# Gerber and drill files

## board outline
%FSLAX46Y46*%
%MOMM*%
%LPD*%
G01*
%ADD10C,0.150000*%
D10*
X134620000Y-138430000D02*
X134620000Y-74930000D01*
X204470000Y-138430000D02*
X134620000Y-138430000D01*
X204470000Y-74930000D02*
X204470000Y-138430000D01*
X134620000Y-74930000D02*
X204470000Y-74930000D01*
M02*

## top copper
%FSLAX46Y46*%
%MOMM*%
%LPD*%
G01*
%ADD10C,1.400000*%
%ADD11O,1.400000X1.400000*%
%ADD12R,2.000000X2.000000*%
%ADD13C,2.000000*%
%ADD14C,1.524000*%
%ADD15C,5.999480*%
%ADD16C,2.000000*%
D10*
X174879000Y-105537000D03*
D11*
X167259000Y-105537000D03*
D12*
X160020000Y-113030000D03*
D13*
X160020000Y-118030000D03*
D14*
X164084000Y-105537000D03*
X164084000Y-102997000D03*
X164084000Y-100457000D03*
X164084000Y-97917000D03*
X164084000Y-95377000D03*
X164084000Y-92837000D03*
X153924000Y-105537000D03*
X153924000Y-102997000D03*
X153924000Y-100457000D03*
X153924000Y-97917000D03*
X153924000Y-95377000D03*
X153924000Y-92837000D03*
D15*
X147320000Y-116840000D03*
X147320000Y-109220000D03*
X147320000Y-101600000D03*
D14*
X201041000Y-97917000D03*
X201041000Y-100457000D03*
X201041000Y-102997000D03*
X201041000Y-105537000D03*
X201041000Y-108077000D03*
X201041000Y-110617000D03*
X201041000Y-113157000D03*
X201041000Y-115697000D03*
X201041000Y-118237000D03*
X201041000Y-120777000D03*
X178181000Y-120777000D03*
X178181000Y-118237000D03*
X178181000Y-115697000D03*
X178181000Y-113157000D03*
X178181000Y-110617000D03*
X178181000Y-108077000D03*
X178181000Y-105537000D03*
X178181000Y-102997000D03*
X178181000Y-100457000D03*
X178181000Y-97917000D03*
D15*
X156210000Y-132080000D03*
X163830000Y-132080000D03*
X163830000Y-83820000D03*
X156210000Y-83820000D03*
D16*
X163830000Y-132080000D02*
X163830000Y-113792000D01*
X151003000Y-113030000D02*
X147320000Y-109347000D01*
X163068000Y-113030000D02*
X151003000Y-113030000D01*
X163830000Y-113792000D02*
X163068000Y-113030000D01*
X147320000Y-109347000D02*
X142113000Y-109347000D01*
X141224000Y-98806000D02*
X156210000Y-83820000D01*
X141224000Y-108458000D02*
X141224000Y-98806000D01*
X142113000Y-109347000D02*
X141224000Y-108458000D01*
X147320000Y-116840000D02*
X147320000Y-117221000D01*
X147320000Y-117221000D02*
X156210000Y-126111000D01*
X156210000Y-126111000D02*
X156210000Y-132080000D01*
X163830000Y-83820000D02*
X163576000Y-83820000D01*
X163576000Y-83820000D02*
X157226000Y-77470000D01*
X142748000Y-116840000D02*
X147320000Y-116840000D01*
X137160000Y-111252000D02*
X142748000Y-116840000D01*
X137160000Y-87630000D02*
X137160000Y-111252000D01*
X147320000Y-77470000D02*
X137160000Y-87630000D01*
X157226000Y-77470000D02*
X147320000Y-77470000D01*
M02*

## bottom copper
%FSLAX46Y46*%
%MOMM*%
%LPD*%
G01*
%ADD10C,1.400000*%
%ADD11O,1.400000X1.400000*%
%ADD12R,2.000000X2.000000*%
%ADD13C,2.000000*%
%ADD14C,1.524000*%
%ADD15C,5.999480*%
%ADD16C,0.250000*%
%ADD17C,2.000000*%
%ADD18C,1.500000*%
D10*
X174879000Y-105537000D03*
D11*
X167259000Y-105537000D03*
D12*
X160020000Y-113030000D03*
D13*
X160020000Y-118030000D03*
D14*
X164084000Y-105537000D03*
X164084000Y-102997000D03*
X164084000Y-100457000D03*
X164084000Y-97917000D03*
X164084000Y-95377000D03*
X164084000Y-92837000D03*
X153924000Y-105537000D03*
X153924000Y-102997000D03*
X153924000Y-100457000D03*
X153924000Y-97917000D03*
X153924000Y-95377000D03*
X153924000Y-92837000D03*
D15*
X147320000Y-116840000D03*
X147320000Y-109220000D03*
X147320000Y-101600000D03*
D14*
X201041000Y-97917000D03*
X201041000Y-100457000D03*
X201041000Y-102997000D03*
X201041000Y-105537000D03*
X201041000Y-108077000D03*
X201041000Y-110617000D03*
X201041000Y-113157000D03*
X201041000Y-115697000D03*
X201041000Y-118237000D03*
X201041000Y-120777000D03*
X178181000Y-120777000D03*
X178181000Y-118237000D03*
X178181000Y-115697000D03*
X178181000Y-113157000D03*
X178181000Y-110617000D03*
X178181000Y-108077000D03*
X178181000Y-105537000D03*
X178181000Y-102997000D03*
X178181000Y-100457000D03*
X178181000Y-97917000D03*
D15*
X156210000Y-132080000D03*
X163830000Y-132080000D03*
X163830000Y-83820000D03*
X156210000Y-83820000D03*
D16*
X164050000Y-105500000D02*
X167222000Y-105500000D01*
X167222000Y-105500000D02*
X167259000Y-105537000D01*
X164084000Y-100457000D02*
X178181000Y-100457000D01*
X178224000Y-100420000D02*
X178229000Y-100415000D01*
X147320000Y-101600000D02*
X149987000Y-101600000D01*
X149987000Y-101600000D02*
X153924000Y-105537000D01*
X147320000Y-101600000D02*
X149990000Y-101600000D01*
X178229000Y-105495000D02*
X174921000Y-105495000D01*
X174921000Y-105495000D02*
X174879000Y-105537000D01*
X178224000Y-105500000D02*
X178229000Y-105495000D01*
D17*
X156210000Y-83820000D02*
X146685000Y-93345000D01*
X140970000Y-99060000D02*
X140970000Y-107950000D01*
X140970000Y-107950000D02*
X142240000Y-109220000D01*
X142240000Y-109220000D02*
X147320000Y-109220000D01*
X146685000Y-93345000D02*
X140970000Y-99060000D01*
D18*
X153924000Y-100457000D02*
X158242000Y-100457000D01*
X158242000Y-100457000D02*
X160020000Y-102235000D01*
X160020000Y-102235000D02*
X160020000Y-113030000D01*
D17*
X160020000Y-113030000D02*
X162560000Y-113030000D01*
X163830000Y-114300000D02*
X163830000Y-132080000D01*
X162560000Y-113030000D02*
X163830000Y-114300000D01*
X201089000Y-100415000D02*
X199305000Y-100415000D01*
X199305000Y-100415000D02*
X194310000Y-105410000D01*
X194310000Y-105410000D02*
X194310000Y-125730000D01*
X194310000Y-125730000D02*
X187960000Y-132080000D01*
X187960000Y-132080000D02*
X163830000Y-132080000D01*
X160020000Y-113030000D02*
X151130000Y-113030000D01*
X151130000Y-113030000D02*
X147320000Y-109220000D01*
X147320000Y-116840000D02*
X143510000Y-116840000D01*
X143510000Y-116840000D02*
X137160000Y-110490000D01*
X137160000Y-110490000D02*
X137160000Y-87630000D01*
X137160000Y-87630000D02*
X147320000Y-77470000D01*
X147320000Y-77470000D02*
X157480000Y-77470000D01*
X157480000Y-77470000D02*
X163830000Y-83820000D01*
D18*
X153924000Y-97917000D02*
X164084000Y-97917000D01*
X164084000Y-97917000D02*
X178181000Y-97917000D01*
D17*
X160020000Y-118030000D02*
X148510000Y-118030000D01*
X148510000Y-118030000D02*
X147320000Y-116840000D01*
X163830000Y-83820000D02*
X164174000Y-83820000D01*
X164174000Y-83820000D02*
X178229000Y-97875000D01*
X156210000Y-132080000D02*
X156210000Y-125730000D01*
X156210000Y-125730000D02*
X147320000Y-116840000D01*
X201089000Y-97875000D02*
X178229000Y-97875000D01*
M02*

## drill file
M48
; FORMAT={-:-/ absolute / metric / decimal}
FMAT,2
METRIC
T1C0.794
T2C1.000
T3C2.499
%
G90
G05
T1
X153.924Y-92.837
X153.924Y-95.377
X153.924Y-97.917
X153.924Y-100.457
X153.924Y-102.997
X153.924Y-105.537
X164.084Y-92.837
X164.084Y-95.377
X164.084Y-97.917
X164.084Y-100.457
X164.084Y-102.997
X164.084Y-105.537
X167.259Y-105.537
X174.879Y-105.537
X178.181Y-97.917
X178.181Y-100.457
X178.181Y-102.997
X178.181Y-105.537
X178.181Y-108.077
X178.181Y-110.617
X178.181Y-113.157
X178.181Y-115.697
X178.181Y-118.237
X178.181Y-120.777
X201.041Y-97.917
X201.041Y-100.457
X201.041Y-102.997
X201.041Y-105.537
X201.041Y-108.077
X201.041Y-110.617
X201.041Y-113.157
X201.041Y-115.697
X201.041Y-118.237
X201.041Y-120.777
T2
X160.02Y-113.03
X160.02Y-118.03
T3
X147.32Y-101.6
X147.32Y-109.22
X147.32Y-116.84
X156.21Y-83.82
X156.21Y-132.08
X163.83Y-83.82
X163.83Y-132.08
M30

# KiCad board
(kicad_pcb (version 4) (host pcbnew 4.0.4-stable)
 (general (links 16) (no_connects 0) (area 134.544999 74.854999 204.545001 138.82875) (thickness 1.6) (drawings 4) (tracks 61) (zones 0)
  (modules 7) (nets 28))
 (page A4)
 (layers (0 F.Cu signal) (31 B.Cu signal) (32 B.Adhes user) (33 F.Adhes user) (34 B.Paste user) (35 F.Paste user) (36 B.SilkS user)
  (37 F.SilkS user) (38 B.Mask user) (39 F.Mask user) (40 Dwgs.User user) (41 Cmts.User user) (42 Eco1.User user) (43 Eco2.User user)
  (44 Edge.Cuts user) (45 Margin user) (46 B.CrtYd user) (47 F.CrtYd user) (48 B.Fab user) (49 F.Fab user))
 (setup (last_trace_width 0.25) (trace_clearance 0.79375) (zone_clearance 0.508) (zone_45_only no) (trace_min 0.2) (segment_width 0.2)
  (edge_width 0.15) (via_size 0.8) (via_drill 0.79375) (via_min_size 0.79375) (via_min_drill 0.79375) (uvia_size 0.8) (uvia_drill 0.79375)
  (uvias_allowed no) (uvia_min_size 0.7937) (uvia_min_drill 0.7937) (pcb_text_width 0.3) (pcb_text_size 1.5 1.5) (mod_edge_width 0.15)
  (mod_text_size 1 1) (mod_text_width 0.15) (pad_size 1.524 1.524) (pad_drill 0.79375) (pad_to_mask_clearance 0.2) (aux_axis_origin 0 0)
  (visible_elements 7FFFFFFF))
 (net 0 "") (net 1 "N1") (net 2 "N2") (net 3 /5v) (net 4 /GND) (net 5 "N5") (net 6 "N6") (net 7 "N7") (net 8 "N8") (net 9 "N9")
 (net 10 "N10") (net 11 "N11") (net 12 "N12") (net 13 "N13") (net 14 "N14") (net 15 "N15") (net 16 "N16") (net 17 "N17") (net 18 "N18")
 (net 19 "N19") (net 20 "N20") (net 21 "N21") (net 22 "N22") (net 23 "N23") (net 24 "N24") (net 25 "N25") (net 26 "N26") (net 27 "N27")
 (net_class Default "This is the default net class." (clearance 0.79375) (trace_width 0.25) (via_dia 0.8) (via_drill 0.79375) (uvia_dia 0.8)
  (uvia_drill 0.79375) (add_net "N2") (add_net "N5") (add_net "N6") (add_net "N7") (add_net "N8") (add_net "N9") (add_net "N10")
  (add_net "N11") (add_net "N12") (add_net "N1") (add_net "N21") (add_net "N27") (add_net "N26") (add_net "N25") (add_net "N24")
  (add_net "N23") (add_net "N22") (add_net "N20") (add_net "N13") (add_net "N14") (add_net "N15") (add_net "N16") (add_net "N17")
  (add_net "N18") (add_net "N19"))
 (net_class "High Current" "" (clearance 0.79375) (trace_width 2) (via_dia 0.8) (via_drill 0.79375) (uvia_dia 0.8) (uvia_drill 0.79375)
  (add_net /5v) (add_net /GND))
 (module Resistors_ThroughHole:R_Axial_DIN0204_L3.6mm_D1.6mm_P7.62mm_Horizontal (layer F.Cu) (at 174.879 105.537 180)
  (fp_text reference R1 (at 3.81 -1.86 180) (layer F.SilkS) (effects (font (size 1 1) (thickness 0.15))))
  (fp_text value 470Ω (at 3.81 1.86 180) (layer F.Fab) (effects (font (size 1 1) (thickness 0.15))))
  (pad 1 thru_hole circle (at 0 0 180) (size 1.4 1.4) (drill 0.79375) (layers *.Cu *.Mask) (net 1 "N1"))
  (pad 2 thru_hole oval (at 7.62 0 180) (size 1.4 1.4) (drill 0.79375) (layers *.Cu *.Mask) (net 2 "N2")))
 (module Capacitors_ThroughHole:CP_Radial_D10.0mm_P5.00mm (layer F.Cu) (at 160.02 113.03 270)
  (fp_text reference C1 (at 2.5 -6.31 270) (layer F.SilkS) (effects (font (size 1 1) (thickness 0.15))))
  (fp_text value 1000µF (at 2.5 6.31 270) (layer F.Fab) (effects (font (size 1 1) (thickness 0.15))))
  (pad 1 thru_hole rect (at 0 0 270) (size 2 2) (drill 1) (layers *.Cu *.Mask) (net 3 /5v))
  (pad 2 thru_hole circle (at 5 0 270) (size 2 2) (drill 1) (layers *.Cu *.Mask) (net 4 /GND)))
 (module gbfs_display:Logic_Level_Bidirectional (layer F.Cu) (at 164.084 105.537 180)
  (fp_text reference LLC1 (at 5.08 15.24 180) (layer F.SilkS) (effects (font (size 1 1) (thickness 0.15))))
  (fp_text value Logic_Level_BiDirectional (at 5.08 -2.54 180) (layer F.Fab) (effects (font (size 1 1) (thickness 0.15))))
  (pad L1 thru_hole circle (at 0 0 180) (size 1.524 1.524) (drill 0.79375) (layers *.Cu *.Mask) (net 2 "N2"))
  (pad L2 thru_hole circle (at 0 2.54 180) (size 1.524 1.524) (drill 0.79375) (layers *.Cu *.Mask) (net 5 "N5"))
  (pad L3 thru_hole circle (at 0 5.08 180) (size 1.524 1.524) (drill 0.79375) (layers *.Cu *.Mask) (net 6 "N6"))
  (pad L4 thru_hole circle (at 0 7.62 180) (size 1.524 1.524) (drill 0.79375) (layers *.Cu *.Mask) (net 4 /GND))
  (pad L5 thru_hole circle (at 0 10.16 180) (size 1.524 1.524) (drill 0.79375) (layers *.Cu *.Mask) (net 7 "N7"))
  (pad L6 thru_hole circle (at 0 12.7 180) (size 1.524 1.524) (drill 0.79375) (layers *.Cu *.Mask) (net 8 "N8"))
  (pad R1 thru_hole circle (at 10.16 0 180) (size 1.524 1.524) (drill 0.79375) (layers *.Cu *.Mask) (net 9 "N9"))
  (pad R2 thru_hole circle (at 10.16 2.54 180) (size 1.524 1.524) (drill 0.79375) (layers *.Cu *.Mask) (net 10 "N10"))
  (pad R3 thru_hole circle (at 10.16 5.08 180) (size 1.524 1.524) (drill 0.79375) (layers *.Cu *.Mask) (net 3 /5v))
  (pad R4 thru_hole circle (at 10.16 7.62 180) (size 1.524 1.524) (drill 0.79375) (layers *.Cu *.Mask) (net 4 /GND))
  (pad R5 thru_hole circle (at 10.16 10.16 180) (size 1.524 1.524) (drill 0.79375) (layers *.Cu *.Mask) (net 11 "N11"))
  (pad R6 thru_hole circle (at 10.16 12.7 180) (size 1.524 1.524) (drill 0.79375) (layers *.Cu *.Mask) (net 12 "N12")))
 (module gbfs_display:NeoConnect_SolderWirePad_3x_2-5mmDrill (layer F.Cu) (at 147.32 109.22 90)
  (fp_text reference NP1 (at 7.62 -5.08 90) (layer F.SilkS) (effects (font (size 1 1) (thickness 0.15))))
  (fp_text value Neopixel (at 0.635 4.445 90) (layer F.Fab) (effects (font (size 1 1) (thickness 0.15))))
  (pad 1 thru_hole circle (at -7.62 0 90) (size 5.99948 5.99948) (drill 2.49936) (layers *.Cu *.Mask) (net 4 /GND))
  (pad 2 thru_hole circle (at 0 0 90) (size 5.99948 5.99948) (drill 2.49936) (layers *.Cu *.Mask) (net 3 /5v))
  (pad 3 thru_hole circle (at 7.62 0 90) (size 5.99948 5.99948) (drill 2.49936) (layers *.Cu *.Mask) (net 9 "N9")))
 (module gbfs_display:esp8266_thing (layer F.Cu) (at 177.927 97.917)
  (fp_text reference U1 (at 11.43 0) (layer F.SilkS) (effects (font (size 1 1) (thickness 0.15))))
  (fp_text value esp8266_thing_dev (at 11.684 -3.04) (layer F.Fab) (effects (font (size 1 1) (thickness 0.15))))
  (pad R1 thru_hole circle (at 23.114 0) (size 1.524 1.524) (drill 0.79375) (layers *.Cu *.Mask) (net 4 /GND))
  (pad R2 thru_hole circle (at 23.114 2.54) (size 1.524 1.524) (drill 0.79375) (layers *.Cu *.Mask) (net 3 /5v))
  (pad R3 thru_hole circle (at 23.114 5.08) (size 1.524 1.524) (drill 0.79375) (layers *.Cu *.Mask) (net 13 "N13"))
  (pad R4 thru_hole circle (at 23.114 7.62) (size 1.524 1.524) (drill 0.79375) (layers *.Cu *.Mask) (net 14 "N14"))
  (pad R5 thru_hole circle (at 23.114 10.16) (size 1.524 1.524) (drill 0.79375) (layers *.Cu *.Mask) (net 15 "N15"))
  (pad R6 thru_hole circle (at 23.114 12.7) (size 1.524 1.524) (drill 0.79375) (layers *.Cu *.Mask) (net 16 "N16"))
  (pad R7 thru_hole circle (at 23.114 15.24) (size 1.524 1.524) (drill 0.79375) (layers *.Cu *.Mask) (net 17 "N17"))
  (pad R8 thru_hole circle (at 23.114 17.78) (size 1.524 1.524) (drill 0.79375) (layers *.Cu *.Mask) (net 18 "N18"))
  (pad R9 thru_hole circle (at 23.114 20.32) (size 1.524 1.524) (drill 0.79375) (layers *.Cu *.Mask) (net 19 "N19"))
  (pad R10 thru_hole circle (at 23.114 22.86) (size 1.524 1.524) (drill 0.79375) (layers *.Cu *.Mask) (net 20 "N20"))
  (pad L10 thru_hole circle (at 0.254 22.86) (size 1.524 1.524) (drill 0.79375) (layers *.Cu *.Mask) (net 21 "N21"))
  (pad L9 thru_hole circle (at 0.254 20.32) (size 1.524 1.524) (drill 0.79375) (layers *.Cu *.Mask) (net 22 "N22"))
  (pad L8 thru_hole circle (at 0.254 17.78) (size 1.524 1.524) (drill 0.79375) (layers *.Cu *.Mask) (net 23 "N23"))
  (pad L7 thru_hole circle (at 0.254 15.24) (size 1.524 1.524) (drill 0.79375) (layers *.Cu *.Mask) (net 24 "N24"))
  (pad L6 thru_hole circle (at 0.254 12.7) (size 1.524 1.524) (drill 0.79375) (layers *.Cu *.Mask) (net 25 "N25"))
  (pad L5 thru_hole circle (at 0.254 10.16) (size 1.524 1.524) (drill 0.79375) (layers *.Cu *.Mask) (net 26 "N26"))
  (pad L4 thru_hole circle (at 0.254 7.62) (size 1.524 1.524) (drill 0.79375) (layers *.Cu *.Mask) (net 1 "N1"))
  (pad L3 thru_hole circle (at 0.254 5.08) (size 1.524 1.524) (drill 0.79375) (layers *.Cu *.Mask) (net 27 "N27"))
  (pad L2 thru_hole circle (at 0.254 2.54) (size 1.524 1.524) (drill 0.79375) (layers *.Cu *.Mask) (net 6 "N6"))
  (pad L1 thru_hole circle (at 0.254 0) (size 1.524 1.524) (drill 0.79375) (layers *.Cu *.Mask) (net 4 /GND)))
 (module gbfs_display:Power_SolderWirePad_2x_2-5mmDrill (layer F.Cu) (at 163.83 132.08)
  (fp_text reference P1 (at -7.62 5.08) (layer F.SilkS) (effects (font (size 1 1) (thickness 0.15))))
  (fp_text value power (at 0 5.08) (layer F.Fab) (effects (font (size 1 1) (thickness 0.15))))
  (pad 1 thru_hole circle (at -7.62 0) (size 5.99948 5.99948) (drill 2.49936) (layers *.Cu *.Mask) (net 4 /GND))
  (pad 2 thru_hole circle (at 0 0) (size 5.99948 5.99948) (drill 2.49936) (layers *.Cu *.Mask) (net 3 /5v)))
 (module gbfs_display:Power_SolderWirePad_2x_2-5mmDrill (layer F.Cu) (at 156.21 83.82 180)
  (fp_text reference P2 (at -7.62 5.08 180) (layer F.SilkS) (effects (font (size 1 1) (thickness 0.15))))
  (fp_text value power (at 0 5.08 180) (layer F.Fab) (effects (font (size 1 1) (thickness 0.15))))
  (pad 1 thru_hole circle (at -7.62 0 180) (size 5.99948 5.99948) (drill 2.49936) (layers *.Cu *.Mask) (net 4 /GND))
  (pad 2 thru_hole circle (at 0 0 180) (size 5.99948 5.99948) (drill 2.49936) (layers *.Cu *.Mask) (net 3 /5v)))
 (gr_line (start 134.62 138.43) (end 134.62 74.93) (angle 90) (layer Edge.Cuts) (width 0.15))
 (gr_line (start 204.47 138.43) (end 134.62 138.43) (angle 90) (layer Edge.Cuts) (width 0.15))
 (gr_line (start 204.47 74.93) (end 204.47 138.43) (angle 90) (layer Edge.Cuts) (width 0.15))
 (gr_line (start 134.62 74.93) (end 204.47 74.93) (angle 90) (layer Edge.Cuts) (width 0.15))
 (segment (start 164.05 105.5) (end 167.222 105.5) (width 0.25) (layer B.Cu) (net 2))
 (segment (start 167.222 105.5) (end 167.259 105.537) (width 0.25) (layer B.Cu) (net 2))
 (segment (start 164.084 100.457) (end 178.181 100.457) (width 0.25) (layer B.Cu) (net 6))
 (segment (start 178.224 100.42) (end 178.229 100.415) (width 0.25) (layer B.Cu) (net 6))
 (segment (start 147.32 101.6) (end 149.987 101.6) (width 0.25) (layer B.Cu) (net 9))
 (segment (start 149.987 101.6) (end 153.924 105.537) (width 0.25) (layer B.Cu) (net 9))
 (segment (start 147.32 101.6) (end 149.99 101.6) (width 0.25) (layer B.Cu) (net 9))
 (segment (start 178.229 105.495) (end 174.921 105.495) (width 0.25) (layer B.Cu) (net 1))
 (segment (start 174.921 105.495) (end 174.879 105.537) (width 0.25) (layer B.Cu) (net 1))
 (segment (start 178.224 105.5) (end 178.229 105.495) (width 0.25) (layer B.Cu) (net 1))
 (segment (start 163.83 132.08) (end 163.83 113.792) (width 2) (layer F.Cu) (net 3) (status 400000))
 (segment (start 151.003 113.03) (end 147.32 109.347) (width 2) (layer F.Cu) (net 3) (status 800000))
 (segment (start 163.068 113.03) (end 151.003 113.03) (width 2) (layer F.Cu) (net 3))
 (segment (start 163.83 113.792) (end 163.068 113.03) (width 2) (layer F.Cu) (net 3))
 (segment (start 147.32 109.347) (end 142.113 109.347) (width 2) (layer F.Cu) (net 3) (status 400000))
 (segment (start 141.224 98.806) (end 156.21 83.82) (width 2) (layer F.Cu) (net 3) (status 800000))
 (segment (start 141.224 108.458) (end 141.224 98.806) (width 2) (layer F.Cu) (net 3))
 (segment (start 142.113 109.347) (end 141.224 108.458) (width 2) (layer F.Cu) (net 3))
 (segment (start 156.21 83.82) (end 146.685 93.345) (width 2) (layer B.Cu) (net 3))
 (segment (start 140.97 99.06) (end 140.97 107.95) (width 2) (layer B.Cu) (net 3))
 (segment (start 140.97 107.95) (end 142.24 109.22) (width 2) (layer B.Cu) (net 3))
 (segment (start 142.24 109.22) (end 147.32 109.22) (width 2) (layer B.Cu) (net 3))
 (segment (start 146.685 93.345) (end 140.97 99.06) (width 2) (layer B.Cu) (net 3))
 (segment (start 153.924 100.457) (end 158.242 100.457) (width 1.5) (layer B.Cu) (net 3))
 (segment (start 158.242 100.457) (end 160.02 102.235) (width 1.5) (layer B.Cu) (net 3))
 (segment (start 160.02 102.235) (end 160.02 113.03) (width 1.5) (layer B.Cu) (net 3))
 (segment (start 160.02 113.03) (end 162.56 113.03) (width 2) (layer B.Cu) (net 3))
 (segment (start 163.83 114.3) (end 163.83 132.08) (width 2) (layer B.Cu) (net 3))
 (segment (start 162.56 113.03) (end 163.83 114.3) (width 2) (layer B.Cu) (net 3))
 (segment (start 201.089 100.415) (end 199.305 100.415) (width 2) (layer B.Cu) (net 3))
 (segment (start 199.305 100.415) (end 194.31 105.41) (width 2) (layer B.Cu) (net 3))
 (segment (start 194.31 105.41) (end 194.31 125.73) (width 2) (layer B.Cu) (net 3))
 (segment (start 194.31 125.73) (end 187.96 132.08) (width 2) (layer B.Cu) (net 3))
 (segment (start 187.96 132.08) (end 163.83 132.08) (width 2) (layer B.Cu) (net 3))
 (segment (start 160.02 113.03) (end 151.13 113.03) (width 2) (layer B.Cu) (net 3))
 (segment (start 151.13 113.03) (end 147.32 109.22) (width 2) (layer B.Cu) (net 3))
 (segment (start 147.32 116.84) (end 147.32 117.221) (width 2) (layer F.Cu) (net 4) (status C00000))
 (segment (start 147.32 117.221) (end 156.21 126.111) (width 2) (layer F.Cu) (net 4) (status 400000))
 (segment (start 156.21 126.111) (end 156.21 132.08) (width 2) (layer F.Cu) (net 4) (status 800000))
 (segment (start 163.83 83.82) (end 163.576 83.82) (width 2) (layer F.Cu) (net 4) (status C00000))
 (segment (start 163.576 83.82) (end 157.226 77.47) (width 2) (layer F.Cu) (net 4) (status 400000))
 (segment (start 142.748 116.84) (end 147.32 116.84) (width 2) (layer F.Cu) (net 4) (status 800000))
 (segment (start 137.16 111.252) (end 142.748 116.84) (width 2) (layer F.Cu) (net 4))
 (segment (start 137.16 87.63) (end 137.16 111.252) (width 2) (layer F.Cu) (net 4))
 (segment (start 147.32 77.47) (end 137.16 87.63) (width 2) (layer F.Cu) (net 4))
 (segment (start 157.226 77.47) (end 147.32 77.47) (width 2) (layer F.Cu) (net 4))
 (segment (start 147.32 116.84) (end 143.51 116.84) (width 2) (layer B.Cu) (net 4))
 (segment (start 143.51 116.84) (end 137.16 110.49) (width 2) (layer B.Cu) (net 4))
 (segment (start 137.16 110.49) (end 137.16 87.63) (width 2) (layer B.Cu) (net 4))
 (segment (start 137.16 87.63) (end 147.32 77.47) (width 2) (layer B.Cu) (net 4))
 (segment (start 147.32 77.47) (end 157.48 77.47) (width 2) (layer B.Cu) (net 4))
 (segment (start 157.48 77.47) (end 163.83 83.82) (width 2) (layer B.Cu) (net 4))
 (segment (start 153.924 97.917) (end 164.084 97.917) (width 1.5) (layer B.Cu) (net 4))
 (segment (start 164.084 97.917) (end 178.181 97.917) (width 1.5) (layer B.Cu) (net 4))
 (segment (start 160.02 118.03) (end 148.51 118.03) (width 2) (layer B.Cu) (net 4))
 (segment (start 148.51 118.03) (end 147.32 116.84) (width 2) (layer B.Cu) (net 4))
 (segment (start 163.83 83.82) (end 164.174 83.82) (width 2) (layer B.Cu) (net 4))
 (segment (start 164.174 83.82) (end 178.229 97.875) (width 2) (layer B.Cu) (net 4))
 (segment (start 156.21 132.08) (end 156.21 125.73) (width 2) (layer B.Cu) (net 4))
 (segment (start 156.21 125.73) (end 147.32 116.84) (width 2) (layer B.Cu) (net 4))
 (segment (start 201.089 97.875) (end 178.229 97.875) (width 2) (layer B.Cu) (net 4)))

